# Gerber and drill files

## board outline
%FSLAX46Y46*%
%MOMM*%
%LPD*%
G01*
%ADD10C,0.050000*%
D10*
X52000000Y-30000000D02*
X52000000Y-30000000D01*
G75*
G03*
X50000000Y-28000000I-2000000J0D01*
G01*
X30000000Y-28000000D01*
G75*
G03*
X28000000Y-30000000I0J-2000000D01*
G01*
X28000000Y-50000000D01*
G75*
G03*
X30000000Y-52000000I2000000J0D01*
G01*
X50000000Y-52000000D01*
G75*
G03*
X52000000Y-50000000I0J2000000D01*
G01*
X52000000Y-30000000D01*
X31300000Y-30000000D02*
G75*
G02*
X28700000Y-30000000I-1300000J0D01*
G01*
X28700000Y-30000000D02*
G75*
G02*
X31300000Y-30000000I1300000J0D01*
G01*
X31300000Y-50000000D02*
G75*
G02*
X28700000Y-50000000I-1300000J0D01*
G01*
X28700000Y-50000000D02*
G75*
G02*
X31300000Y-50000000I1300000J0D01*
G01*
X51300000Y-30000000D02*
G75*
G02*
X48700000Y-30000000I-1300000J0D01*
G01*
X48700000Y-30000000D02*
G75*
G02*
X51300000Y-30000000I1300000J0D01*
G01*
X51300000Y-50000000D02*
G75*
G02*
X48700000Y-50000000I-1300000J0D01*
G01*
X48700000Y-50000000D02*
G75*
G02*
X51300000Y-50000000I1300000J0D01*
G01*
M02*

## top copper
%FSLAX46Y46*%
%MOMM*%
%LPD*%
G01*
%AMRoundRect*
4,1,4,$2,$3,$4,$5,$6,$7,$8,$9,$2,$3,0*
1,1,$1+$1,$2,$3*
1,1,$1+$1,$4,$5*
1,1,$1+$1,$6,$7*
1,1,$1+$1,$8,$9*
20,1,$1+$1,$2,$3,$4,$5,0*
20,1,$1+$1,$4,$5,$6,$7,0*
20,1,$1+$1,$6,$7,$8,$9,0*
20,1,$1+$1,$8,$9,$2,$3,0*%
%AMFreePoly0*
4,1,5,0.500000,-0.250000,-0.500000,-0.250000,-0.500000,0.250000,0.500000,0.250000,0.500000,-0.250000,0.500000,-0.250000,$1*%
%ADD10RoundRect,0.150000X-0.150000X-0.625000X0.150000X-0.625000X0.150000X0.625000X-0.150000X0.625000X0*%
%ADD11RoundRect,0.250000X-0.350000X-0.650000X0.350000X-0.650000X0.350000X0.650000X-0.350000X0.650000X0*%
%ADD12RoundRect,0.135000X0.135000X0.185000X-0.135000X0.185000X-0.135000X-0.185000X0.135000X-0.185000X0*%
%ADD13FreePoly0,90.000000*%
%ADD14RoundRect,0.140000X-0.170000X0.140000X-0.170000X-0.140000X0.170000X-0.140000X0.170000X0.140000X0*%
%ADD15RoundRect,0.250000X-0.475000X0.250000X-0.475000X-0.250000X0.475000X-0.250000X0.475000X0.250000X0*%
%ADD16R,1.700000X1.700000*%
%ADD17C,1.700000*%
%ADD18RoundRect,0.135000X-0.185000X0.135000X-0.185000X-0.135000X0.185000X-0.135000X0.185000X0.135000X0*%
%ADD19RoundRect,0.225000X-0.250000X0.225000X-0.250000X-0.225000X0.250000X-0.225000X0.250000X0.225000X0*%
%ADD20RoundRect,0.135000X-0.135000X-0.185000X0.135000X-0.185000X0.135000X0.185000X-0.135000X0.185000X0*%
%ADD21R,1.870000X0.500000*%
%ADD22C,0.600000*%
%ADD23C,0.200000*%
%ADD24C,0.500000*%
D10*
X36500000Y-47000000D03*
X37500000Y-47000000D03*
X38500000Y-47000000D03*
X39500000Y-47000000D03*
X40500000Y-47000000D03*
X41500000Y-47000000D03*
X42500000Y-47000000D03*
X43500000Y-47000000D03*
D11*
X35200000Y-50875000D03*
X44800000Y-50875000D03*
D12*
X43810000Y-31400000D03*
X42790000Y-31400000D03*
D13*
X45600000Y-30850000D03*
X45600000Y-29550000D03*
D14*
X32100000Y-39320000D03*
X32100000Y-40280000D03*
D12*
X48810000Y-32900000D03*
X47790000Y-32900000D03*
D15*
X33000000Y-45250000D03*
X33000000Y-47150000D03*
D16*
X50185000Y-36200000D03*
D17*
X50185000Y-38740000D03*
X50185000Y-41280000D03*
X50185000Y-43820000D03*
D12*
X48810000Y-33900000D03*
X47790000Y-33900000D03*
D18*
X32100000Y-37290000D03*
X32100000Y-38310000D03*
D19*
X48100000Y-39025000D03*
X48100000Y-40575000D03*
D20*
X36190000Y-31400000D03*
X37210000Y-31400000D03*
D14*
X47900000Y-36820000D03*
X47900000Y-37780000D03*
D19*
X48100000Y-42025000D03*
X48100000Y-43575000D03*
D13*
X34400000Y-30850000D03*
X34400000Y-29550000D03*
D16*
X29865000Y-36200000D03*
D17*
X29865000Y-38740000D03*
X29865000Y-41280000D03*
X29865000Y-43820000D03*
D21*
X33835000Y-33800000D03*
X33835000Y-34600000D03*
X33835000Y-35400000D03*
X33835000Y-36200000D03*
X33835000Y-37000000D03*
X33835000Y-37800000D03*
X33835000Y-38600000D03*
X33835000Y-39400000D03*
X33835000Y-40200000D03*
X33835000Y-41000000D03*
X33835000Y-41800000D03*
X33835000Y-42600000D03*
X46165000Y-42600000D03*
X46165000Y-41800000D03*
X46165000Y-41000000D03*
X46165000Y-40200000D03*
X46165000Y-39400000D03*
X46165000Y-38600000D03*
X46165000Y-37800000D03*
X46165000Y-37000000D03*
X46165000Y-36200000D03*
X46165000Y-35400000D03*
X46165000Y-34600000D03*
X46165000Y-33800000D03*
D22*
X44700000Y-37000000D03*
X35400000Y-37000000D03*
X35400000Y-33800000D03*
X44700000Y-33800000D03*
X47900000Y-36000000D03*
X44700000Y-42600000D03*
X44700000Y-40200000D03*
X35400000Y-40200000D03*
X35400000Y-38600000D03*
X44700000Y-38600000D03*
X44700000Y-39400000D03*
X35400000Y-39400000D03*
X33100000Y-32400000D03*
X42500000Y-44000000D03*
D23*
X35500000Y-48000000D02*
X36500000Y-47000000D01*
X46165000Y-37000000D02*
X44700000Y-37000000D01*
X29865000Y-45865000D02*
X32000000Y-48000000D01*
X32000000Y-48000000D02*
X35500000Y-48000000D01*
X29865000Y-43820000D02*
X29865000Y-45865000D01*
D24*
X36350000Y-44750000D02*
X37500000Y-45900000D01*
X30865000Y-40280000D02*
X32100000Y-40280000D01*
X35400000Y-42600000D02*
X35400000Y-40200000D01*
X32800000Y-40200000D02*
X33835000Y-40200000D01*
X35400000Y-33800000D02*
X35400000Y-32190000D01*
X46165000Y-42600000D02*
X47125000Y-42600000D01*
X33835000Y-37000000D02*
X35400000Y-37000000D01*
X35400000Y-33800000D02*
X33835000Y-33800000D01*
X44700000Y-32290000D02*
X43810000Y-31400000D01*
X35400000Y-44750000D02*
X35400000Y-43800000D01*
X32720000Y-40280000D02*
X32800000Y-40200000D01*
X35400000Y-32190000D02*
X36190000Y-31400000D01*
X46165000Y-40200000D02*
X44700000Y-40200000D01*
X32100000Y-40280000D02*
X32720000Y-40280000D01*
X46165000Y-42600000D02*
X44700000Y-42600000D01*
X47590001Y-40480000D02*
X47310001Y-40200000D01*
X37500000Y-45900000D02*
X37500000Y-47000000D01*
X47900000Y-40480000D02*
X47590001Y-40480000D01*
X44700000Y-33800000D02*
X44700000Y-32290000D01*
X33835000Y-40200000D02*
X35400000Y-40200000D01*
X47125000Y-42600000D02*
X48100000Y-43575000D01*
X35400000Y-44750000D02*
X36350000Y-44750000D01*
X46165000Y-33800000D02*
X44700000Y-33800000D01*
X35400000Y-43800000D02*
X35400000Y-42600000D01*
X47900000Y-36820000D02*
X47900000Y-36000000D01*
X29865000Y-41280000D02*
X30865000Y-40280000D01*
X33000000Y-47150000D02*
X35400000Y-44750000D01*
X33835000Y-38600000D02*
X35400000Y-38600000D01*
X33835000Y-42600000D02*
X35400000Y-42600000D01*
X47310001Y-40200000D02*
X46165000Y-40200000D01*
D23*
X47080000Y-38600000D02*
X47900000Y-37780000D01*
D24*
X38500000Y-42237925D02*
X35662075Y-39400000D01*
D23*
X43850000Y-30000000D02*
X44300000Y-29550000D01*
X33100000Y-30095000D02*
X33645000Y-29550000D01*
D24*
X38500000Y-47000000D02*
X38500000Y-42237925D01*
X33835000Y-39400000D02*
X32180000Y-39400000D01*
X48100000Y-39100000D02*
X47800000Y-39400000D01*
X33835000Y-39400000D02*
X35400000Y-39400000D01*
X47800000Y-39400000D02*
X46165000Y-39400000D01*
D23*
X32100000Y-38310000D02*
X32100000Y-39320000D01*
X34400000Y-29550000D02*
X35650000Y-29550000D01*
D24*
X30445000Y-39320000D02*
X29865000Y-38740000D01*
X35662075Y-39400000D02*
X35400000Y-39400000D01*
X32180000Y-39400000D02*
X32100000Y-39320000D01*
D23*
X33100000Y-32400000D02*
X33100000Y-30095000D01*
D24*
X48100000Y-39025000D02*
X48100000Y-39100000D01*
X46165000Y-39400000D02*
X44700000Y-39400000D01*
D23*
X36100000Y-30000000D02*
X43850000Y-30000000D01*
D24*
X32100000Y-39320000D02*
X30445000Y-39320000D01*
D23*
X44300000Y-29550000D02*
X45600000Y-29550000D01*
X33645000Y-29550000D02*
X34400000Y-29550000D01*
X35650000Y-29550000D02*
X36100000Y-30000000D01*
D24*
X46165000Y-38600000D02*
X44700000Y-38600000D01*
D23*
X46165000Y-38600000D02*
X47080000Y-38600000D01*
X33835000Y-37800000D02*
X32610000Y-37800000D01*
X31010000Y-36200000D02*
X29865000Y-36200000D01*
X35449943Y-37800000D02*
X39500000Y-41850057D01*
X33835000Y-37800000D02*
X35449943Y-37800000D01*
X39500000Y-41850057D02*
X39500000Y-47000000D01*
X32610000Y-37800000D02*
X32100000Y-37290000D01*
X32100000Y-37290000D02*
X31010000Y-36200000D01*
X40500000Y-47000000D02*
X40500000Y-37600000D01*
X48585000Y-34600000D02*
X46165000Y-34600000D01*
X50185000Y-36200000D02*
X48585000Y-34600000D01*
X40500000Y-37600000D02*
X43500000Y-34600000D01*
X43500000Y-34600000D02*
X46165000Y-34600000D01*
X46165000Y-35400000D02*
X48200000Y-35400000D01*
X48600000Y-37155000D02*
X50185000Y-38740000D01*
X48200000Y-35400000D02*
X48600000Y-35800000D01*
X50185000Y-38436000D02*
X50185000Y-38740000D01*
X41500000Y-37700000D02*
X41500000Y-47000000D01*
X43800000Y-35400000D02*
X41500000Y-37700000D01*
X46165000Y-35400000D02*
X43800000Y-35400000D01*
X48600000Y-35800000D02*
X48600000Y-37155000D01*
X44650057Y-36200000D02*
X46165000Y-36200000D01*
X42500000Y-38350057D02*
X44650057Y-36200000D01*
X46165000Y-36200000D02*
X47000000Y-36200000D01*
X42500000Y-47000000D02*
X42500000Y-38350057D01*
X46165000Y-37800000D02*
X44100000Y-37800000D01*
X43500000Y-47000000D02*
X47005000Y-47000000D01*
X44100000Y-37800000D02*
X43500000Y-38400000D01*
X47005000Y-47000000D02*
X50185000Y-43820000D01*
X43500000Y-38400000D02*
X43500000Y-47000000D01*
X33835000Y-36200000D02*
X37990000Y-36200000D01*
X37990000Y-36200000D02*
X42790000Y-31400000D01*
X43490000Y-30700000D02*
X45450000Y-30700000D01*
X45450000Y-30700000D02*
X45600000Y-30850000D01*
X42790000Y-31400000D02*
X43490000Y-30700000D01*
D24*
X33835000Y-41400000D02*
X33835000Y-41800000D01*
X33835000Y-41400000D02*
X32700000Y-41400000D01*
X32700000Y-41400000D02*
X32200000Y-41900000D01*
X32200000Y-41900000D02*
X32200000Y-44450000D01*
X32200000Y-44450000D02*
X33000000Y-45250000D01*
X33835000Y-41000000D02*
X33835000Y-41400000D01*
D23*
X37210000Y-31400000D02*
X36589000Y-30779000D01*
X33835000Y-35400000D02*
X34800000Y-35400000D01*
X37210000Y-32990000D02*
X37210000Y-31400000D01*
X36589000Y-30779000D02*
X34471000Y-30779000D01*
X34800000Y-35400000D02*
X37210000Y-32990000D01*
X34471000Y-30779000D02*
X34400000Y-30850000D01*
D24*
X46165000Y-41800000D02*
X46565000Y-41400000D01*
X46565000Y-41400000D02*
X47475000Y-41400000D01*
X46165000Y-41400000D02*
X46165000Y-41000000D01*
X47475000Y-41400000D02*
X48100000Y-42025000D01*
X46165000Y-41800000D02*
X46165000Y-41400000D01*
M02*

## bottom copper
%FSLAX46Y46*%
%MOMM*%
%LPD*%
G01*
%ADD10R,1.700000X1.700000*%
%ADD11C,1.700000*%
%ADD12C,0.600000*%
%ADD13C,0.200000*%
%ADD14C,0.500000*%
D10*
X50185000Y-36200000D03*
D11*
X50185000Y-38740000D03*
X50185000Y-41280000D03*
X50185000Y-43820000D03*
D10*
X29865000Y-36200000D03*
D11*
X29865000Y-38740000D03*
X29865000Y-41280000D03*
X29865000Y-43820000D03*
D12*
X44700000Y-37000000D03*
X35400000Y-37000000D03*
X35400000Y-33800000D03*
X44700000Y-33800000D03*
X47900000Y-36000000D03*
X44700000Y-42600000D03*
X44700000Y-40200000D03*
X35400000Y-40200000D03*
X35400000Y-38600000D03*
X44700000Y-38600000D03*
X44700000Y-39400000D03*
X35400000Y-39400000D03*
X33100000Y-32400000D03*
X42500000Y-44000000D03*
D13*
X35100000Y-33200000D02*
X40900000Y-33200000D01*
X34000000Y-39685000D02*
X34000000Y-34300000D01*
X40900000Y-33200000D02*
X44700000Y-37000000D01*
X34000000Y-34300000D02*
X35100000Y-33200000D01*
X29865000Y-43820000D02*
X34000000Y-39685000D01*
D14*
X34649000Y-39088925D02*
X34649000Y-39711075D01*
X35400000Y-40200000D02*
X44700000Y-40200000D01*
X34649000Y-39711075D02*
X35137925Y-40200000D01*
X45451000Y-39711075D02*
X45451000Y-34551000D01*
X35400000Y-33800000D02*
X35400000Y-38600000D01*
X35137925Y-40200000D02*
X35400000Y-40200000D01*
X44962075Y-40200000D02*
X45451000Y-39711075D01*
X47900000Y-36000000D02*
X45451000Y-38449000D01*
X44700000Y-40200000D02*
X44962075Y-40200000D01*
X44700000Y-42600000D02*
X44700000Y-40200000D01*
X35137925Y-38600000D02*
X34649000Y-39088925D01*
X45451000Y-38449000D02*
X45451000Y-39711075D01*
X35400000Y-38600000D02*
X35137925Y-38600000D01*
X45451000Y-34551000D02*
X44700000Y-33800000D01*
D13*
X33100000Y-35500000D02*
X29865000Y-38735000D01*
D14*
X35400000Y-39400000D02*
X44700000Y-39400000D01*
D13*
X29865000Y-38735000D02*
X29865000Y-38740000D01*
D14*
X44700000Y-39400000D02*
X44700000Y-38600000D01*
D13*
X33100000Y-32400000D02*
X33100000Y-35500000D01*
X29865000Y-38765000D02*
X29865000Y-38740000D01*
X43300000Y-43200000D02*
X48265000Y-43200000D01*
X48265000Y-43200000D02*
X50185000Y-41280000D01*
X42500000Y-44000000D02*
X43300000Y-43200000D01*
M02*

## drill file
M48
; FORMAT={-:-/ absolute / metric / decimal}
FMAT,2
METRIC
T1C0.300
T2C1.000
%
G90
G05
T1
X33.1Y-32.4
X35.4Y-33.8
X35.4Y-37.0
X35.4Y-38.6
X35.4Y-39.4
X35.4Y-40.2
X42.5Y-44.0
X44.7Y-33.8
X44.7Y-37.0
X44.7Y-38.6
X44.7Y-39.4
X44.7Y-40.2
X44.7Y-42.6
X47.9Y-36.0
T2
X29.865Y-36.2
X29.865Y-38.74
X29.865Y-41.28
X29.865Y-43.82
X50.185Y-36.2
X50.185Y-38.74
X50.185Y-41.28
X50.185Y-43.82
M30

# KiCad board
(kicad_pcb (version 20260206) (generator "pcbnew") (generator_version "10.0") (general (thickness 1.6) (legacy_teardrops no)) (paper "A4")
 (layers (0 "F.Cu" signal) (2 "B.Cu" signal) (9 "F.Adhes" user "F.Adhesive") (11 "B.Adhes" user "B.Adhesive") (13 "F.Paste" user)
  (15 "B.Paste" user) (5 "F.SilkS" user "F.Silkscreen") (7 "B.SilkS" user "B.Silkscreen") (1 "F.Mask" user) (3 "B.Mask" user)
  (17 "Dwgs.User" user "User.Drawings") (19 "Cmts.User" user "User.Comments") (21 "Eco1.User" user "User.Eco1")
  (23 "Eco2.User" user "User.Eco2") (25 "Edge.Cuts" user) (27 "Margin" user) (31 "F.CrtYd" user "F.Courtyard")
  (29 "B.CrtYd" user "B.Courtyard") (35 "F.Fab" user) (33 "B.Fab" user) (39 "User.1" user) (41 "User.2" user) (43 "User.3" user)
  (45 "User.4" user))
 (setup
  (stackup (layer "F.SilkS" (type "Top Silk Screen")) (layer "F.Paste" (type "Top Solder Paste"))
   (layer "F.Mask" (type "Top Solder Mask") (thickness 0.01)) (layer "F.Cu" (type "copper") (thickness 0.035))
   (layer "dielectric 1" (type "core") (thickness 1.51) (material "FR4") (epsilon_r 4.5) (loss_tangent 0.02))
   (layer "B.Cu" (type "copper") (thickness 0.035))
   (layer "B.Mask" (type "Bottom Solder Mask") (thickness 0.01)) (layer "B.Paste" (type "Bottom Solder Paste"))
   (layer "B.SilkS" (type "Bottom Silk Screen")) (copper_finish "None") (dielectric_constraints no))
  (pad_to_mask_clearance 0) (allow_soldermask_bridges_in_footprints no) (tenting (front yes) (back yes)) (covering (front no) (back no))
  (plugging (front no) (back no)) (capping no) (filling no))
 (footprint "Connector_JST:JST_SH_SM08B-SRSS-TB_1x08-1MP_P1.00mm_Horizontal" (layer "F.Cu") (at 40 49)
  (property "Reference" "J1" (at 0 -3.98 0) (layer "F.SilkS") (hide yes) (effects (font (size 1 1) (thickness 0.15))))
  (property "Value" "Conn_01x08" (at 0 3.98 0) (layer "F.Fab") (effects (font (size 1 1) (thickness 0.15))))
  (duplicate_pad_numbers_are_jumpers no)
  (pad "1" smd roundrect (at -3.5 -2) (size 0.6 1.55) (layers "F.Cu" "F.Mask" "F.Paste") (roundrect_rratio 0.25) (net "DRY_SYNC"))
  (pad "2" smd roundrect (at -2.5 -2) (size 0.6 1.55) (layers "F.Cu" "F.Mask" "F.Paste") (roundrect_rratio 0.25) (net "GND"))
  (pad "3" smd roundrect (at -1.5 -2) (size 0.6 1.55) (layers "F.Cu" "F.Mask" "F.Paste") (roundrect_rratio 0.25) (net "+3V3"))
  (pad "4" smd roundrect (at -0.5 -2) (size 0.6 1.55) (layers "F.Cu" "F.Mask" "F.Paste") (roundrect_rratio 0.25) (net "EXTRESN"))
  (pad "5" smd roundrect (at 0.5 -2) (size 0.6 1.55) (layers "F.Cu" "F.Mask" "F.Paste") (roundrect_rratio 0.25) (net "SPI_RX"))
  (pad "6" smd roundrect (at 1.5 -2) (size 0.6 1.55) (layers "F.Cu" "F.Mask" "F.Paste") (roundrect_rratio 0.25) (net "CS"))
  (pad "7" smd roundrect (at 2.5 -2) (size 0.6 1.55) (layers "F.Cu" "F.Mask" "F.Paste") (roundrect_rratio 0.25) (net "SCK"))
  (pad "8" smd roundrect (at 3.5 -2) (size 0.6 1.55) (layers "F.Cu" "F.Mask" "F.Paste") (roundrect_rratio 0.25) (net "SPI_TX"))
  (pad "MP" smd roundrect (at -4.8 1.875) (size 1.2 1.8) (layers "F.Cu" "F.Mask" "F.Paste") (roundrect_rratio 0.208333))
  (pad "MP" smd roundrect (at 4.8 1.875) (size 1.2 1.8) (layers "F.Cu" "F.Mask" "F.Paste") (roundrect_rratio 0.208333)))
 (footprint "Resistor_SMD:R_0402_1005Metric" (layer "F.Cu") (at 43.3 31.4 180)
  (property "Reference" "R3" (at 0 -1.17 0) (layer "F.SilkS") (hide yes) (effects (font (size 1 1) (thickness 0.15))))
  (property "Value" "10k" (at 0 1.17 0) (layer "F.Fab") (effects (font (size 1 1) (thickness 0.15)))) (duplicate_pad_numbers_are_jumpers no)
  (pad "1" smd roundrect (at -0.51 0 180) (size 0.54 0.64) (layers "F.Cu" "F.Mask" "F.Paste") (roundrect_rratio 0.25) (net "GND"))
  (pad "2" smd roundrect (at 0.51 0 180) (size 0.54 0.64) (layers "F.Cu" "F.Mask" "F.Paste") (roundrect_rratio 0.25) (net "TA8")))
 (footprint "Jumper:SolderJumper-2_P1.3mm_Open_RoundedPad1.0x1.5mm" (layer "F.Cu") (at 45.6 30.2 90)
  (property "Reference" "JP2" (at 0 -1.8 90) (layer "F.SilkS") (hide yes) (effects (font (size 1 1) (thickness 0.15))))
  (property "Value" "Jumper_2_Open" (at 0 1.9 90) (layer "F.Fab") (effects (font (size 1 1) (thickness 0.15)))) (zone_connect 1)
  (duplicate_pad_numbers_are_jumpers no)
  (pad "1" smd custom (at -0.65 0 90) (size 1 0.5) (layers "F.Cu" "F.Mask") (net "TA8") (zone_connect 2) (thermal_bridge_angle 45)
   (options (clearance outline) (anchor rect)) (primitives))
  (pad "2" smd custom (at 0.65 0 90) (size 1 0.5) (layers "F.Cu" "F.Mask") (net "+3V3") (zone_connect 2) (thermal_bridge_angle 45)
   (options (clearance outline) (anchor rect)) (primitives)))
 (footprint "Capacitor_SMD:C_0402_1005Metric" (layer "F.Cu") (at 32.1 39.8 -90)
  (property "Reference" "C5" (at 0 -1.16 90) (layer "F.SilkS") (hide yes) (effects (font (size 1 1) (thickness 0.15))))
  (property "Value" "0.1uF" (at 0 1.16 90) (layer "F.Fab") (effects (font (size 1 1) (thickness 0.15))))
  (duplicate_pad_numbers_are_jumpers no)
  (pad "1" smd roundrect (at -0.48 0 270) (size 0.56 0.62) (layers "F.Cu" "F.Mask" "F.Paste") (roundrect_rratio 0.25) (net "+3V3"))
  (pad "2" smd roundrect (at 0.48 0 270) (size 0.56 0.62) (layers "F.Cu" "F.Mask" "F.Paste") (roundrect_rratio 0.25) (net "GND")))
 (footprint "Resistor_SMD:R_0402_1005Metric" (layer "F.Cu") (at 48.3 32.9 180)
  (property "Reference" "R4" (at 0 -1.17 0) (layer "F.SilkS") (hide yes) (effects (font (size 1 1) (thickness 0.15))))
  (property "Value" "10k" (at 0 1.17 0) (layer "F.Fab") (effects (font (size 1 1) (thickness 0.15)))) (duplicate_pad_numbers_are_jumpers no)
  (pad "1" smd roundrect (at -0.51 0 180) (size 0.54 0.64) (layers "F.Cu" "F.Mask" "F.Paste") (roundrect_rratio 0.25)
   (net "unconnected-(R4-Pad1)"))
  (pad "2" smd roundrect (at 0.51 0 180) (size 0.54 0.64) (layers "F.Cu" "F.Mask" "F.Paste") (roundrect_rratio 0.25)
   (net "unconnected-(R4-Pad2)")))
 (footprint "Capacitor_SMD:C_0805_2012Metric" (layer "F.Cu") (at 33 46.2 -90)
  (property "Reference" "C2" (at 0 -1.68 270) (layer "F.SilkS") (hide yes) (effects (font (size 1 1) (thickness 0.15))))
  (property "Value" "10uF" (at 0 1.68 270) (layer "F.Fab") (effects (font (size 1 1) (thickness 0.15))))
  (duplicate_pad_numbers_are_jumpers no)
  (pad "1" smd roundrect (at -0.95 0 270) (size 1 1.45) (layers "F.Cu" "F.Mask" "F.Paste") (roundrect_rratio 0.25) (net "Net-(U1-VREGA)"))
  (pad "2" smd roundrect (at 0.95 0 270) (size 1 1.45) (layers "F.Cu" "F.Mask" "F.Paste") (roundrect_rratio 0.25) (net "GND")))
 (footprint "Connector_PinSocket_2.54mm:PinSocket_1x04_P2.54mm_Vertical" (layer "F.Cu") (at 50.185 36.2)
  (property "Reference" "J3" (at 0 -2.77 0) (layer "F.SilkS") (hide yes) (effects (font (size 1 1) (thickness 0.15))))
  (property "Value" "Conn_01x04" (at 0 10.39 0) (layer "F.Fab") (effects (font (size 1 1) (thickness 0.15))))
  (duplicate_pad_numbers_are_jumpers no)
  (pad "1" thru_hole rect (at 0 0) (size 1.7 1.7) (drill 1) (layers "*.Cu" "*.Mask") (remove_unused_layers no) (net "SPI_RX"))
  (pad "2" thru_hole circle (at 0 2.54) (size 1.7 1.7) (drill 1) (layers "*.Cu" "*.Mask") (remove_unused_layers no) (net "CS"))
  (pad "3" thru_hole circle (at 0 5.08) (size 1.7 1.7) (drill 1) (layers "*.Cu" "*.Mask") (remove_unused_layers no) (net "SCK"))
  (pad "4" thru_hole circle (at 0 7.62) (size 1.7 1.7) (drill 1) (layers "*.Cu" "*.Mask") (remove_unused_layers no) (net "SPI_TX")))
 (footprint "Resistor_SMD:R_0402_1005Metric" (layer "F.Cu") (at 48.3 33.9 180)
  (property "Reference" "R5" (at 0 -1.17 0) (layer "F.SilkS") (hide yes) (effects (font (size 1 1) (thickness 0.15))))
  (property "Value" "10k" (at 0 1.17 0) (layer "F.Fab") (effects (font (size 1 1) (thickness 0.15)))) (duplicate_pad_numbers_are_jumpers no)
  (pad "1" smd roundrect (at -0.51 0 180) (size 0.54 0.64) (layers "F.Cu" "F.Mask" "F.Paste") (roundrect_rratio 0.25)
   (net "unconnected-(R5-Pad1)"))
  (pad "2" smd roundrect (at 0.51 0 180) (size 0.54 0.64) (layers "F.Cu" "F.Mask" "F.Paste") (roundrect_rratio 0.25)
   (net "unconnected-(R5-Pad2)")))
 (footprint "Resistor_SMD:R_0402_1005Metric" (layer "F.Cu") (at 32.1 37.8 -90)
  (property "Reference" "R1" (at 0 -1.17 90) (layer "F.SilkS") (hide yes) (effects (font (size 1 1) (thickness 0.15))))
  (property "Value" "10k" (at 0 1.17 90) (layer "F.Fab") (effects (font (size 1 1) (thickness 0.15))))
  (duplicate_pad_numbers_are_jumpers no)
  (pad "1" smd roundrect (at -0.51 0 270) (size 0.54 0.64) (layers "F.Cu" "F.Mask" "F.Paste") (roundrect_rratio 0.25) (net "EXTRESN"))
  (pad "2" smd roundrect (at 0.51 0 270) (size 0.54 0.64) (layers "F.Cu" "F.Mask" "F.Paste") (roundrect_rratio 0.25) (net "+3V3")))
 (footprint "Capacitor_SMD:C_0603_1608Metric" (layer "F.Cu") (at 48.1 39.8 -90)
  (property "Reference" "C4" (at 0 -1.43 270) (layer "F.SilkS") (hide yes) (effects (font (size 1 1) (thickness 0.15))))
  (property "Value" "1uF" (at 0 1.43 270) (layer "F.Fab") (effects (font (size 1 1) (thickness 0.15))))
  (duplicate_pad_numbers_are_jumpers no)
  (pad "1" smd roundrect (at -0.775 0 270) (size 0.9 0.95) (layers "F.Cu" "F.Mask" "F.Paste") (roundrect_rratio 0.25) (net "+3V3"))
  (pad "2" smd roundrect (at 0.775 0 270) (size 0.9 0.95) (layers "F.Cu" "F.Mask" "F.Paste") (roundrect_rratio 0.25) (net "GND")))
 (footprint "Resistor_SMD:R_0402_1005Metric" (layer "F.Cu") (at 36.7 31.4)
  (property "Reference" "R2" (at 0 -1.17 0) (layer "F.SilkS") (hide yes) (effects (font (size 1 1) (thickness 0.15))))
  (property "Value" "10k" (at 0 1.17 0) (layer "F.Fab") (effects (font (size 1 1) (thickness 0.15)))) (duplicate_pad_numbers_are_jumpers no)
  (pad "1" smd roundrect (at -0.51 0) (size 0.54 0.64) (layers "F.Cu" "F.Mask" "F.Paste") (roundrect_rratio 0.25) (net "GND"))
  (pad "2" smd roundrect (at 0.51 0) (size 0.54 0.64) (layers "F.Cu" "F.Mask" "F.Paste") (roundrect_rratio 0.25) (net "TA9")))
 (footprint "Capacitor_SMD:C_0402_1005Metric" (layer "F.Cu") (at 47.9 37.3 -90)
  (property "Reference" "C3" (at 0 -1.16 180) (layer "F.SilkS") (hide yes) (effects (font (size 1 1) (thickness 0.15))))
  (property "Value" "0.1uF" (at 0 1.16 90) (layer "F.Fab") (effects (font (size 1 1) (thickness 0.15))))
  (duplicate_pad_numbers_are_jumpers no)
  (pad "1" smd roundrect (at -0.48 0 270) (size 0.56 0.62) (layers "F.Cu" "F.Mask" "F.Paste") (roundrect_rratio 0.25) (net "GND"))
  (pad "2" smd roundrect (at 0.48 0 270) (size 0.56 0.62) (layers "F.Cu" "F.Mask" "F.Paste") (roundrect_rratio 0.25) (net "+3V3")))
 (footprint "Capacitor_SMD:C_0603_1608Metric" (layer "F.Cu") (at 48.1 42.8 -90)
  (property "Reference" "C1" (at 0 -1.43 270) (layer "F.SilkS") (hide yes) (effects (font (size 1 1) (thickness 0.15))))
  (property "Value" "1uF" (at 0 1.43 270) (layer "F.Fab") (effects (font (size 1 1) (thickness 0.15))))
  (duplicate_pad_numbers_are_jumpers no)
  (pad "1" smd roundrect (at -0.775 0 270) (size 0.9 0.95) (layers "F.Cu" "F.Mask" "F.Paste") (roundrect_rratio 0.25) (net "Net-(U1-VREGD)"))
  (pad "2" smd roundrect (at 0.775 0 270) (size 0.9 0.95) (layers "F.Cu" "F.Mask" "F.Paste") (roundrect_rratio 0.25) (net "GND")))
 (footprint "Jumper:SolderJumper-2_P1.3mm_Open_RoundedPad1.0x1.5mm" (layer "F.Cu") (at 34.4 30.2 90)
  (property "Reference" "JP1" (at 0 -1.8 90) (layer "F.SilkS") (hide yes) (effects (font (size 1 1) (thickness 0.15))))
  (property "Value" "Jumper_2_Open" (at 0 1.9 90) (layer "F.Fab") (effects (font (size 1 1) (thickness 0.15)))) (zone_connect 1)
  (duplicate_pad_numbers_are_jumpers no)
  (pad "1" smd custom (at -0.65 0 90) (size 1 0.5) (layers "F.Cu" "F.Mask") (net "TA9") (zone_connect 2) (thermal_bridge_angle 45)
   (options (clearance outline) (anchor rect)) (primitives))
  (pad "2" smd custom (at 0.65 0 90) (size 1 0.5) (layers "F.Cu" "F.Mask") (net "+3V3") (zone_connect 2) (thermal_bridge_angle 45)
   (options (clearance outline) (anchor rect)) (primitives)))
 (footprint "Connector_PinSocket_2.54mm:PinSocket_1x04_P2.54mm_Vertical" (layer "F.Cu") (at 29.865 36.2)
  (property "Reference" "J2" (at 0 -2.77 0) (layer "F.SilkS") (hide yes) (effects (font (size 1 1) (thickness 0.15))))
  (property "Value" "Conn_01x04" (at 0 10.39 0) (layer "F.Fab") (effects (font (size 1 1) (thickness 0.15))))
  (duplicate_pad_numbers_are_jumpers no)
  (pad "1" thru_hole rect (at 0 0) (size 1.7 1.7) (drill 1) (layers "*.Cu" "*.Mask") (remove_unused_layers no) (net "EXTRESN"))
  (pad "2" thru_hole circle (at 0 2.54) (size 1.7 1.7) (drill 1) (layers "*.Cu" "*.Mask") (remove_unused_layers no) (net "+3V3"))
  (pad "3" thru_hole circle (at 0 5.08) (size 1.7 1.7) (drill 1) (layers "*.Cu" "*.Mask") (remove_unused_layers no) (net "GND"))
  (pad "4" thru_hole circle (at 0 7.62) (size 1.7 1.7) (drill 1) (layers "*.Cu" "*.Mask") (remove_unused_layers no) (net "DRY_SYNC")))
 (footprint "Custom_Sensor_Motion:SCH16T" (layer "F.Cu") (at 40 38.2)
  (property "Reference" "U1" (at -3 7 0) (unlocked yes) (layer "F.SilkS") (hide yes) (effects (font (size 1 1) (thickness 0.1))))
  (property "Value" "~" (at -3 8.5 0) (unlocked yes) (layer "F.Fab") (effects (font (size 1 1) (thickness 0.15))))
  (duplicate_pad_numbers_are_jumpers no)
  (pad "1" smd rect (at -6.165 -4.4) (size 1.87 0.5) (layers "F.Cu" "F.Mask" "F.Paste") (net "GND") (thermal_bridge_angle 45))
  (pad "2" smd rect (at -6.165 -3.6) (size 1.87 0.5) (layers "F.Cu" "F.Mask" "F.Paste") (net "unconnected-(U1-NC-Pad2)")
   (thermal_bridge_angle 45))
  (pad "3" smd rect (at -6.165 -2.8) (size 1.87 0.5) (layers "F.Cu" "F.Mask" "F.Paste") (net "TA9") (thermal_bridge_angle 45))
  (pad "4" smd rect (at -6.165 -2) (size 1.87 0.5) (layers "F.Cu" "F.Mask" "F.Paste") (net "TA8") (thermal_bridge_angle 45))
  (pad "5" smd rect (at -6.165 -1.2) (size 1.87 0.5) (layers "F.Cu" "F.Mask" "F.Paste") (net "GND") (thermal_bridge_angle 45))
  (pad "6" smd rect (at -6.165 -0.4) (size 1.87 0.5) (layers "F.Cu" "F.Mask" "F.Paste") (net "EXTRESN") (thermal_bridge_angle 45))
  (pad "7" smd rect (at -6.165 0.4) (size 1.87 0.5) (layers "F.Cu" "F.Mask" "F.Paste") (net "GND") (thermal_bridge_angle 45))
  (pad "8" smd rect (at -6.165 1.2) (size 1.87 0.5) (layers "F.Cu" "F.Mask" "F.Paste") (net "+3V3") (thermal_bridge_angle 45))
  (pad "9" smd rect (at -6.165 2) (size 1.87 0.5) (layers "F.Cu" "F.Mask" "F.Paste") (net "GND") (thermal_bridge_angle 45))
  (pad "10" smd rect (at -6.165 2.8) (size 1.87 0.5) (layers "F.Cu" "F.Mask" "F.Paste") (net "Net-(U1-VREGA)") (thermal_bridge_angle 45))
  (pad "11" smd rect (at -6.165 3.6) (size 1.87 0.5) (layers "F.Cu" "F.Mask" "F.Paste") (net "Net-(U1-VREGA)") (thermal_bridge_angle 45))
  (pad "12" smd rect (at -6.165 4.4) (size 1.87 0.5) (layers "F.Cu" "F.Mask" "F.Paste") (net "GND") (thermal_bridge_angle 45))
  (pad "13" smd rect (at 6.165 4.4) (size 1.87 0.5) (layers "F.Cu" "F.Mask" "F.Paste") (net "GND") (thermal_bridge_angle 45))
  (pad "14" smd rect (at 6.165 3.6) (size 1.87 0.5) (layers "F.Cu" "F.Mask" "F.Paste") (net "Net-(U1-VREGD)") (thermal_bridge_angle 45))
  (pad "15" smd rect (at 6.165 2.8) (size 1.87 0.5) (layers "F.Cu" "F.Mask" "F.Paste") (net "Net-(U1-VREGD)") (thermal_bridge_angle 45))
  (pad "16" smd rect (at 6.165 2) (size 1.87 0.5) (layers "F.Cu" "F.Mask" "F.Paste") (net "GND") (thermal_bridge_angle 45))
  (pad "17" smd rect (at 6.165 1.2) (size 1.87 0.5) (layers "F.Cu" "F.Mask" "F.Paste") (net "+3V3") (thermal_bridge_angle 45))
  (pad "18" smd rect (at 6.165 0.4) (size 1.87 0.5) (layers "F.Cu" "F.Mask" "F.Paste") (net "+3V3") (thermal_bridge_angle 45))
  (pad "19" smd rect (at 6.165 -0.4) (size 1.87 0.5) (layers "F.Cu" "F.Mask" "F.Paste") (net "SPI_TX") (thermal_bridge_angle 45))
  (pad "20" smd rect (at 6.165 -1.2) (size 1.87 0.5) (layers "F.Cu" "F.Mask" "F.Paste") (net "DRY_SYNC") (thermal_bridge_angle 45))
  (pad "21" smd rect (at 6.165 -2) (size 1.87 0.5) (layers "F.Cu" "F.Mask" "F.Paste") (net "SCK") (thermal_bridge_angle 45))
  (pad "22" smd rect (at 6.165 -2.8) (size 1.87 0.5) (layers "F.Cu" "F.Mask" "F.Paste") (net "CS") (thermal_bridge_angle 45))
  (pad "23" smd rect (at 6.165 -3.6) (size 1.87 0.5) (layers "F.Cu" "F.Mask" "F.Paste") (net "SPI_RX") (thermal_bridge_angle 45))
  (pad "24" smd rect (at 6.165 -4.4) (size 1.87 0.5) (layers "F.Cu" "F.Mask" "F.Paste") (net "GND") (thermal_bridge_angle 45)))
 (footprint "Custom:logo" (layer "B.Cu") (at 40 32 180)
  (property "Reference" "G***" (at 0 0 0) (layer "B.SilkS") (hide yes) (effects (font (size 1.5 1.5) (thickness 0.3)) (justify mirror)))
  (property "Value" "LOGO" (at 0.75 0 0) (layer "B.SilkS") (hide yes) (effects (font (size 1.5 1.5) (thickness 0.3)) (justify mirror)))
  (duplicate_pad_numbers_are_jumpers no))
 (gr_poly
  (pts (arc (start 52 30) (mid 51.414214 28.585786) (end 50 28)) (arc (start 30 28) (mid 28.585786 28.585786) (end 28 30))
   (arc (start 28 50) (mid 28.585786 51.414214) (end 30 52)) (arc (start 50 52) (mid 51.414214 51.414214) (end 52 50)))
  (stroke (width 0.05) (type solid)) (fill no) (layer "Edge.Cuts"))
 (gr_circle (center 30 30) (end 31.3 30) (stroke (width 0.05) (type solid)) (fill no) (layer "Edge.Cuts"))
 (gr_circle (center 30 50) (end 31.3 50) (stroke (width 0.05) (type solid)) (fill no) (layer "Edge.Cuts"))
 (gr_circle (center 50 30) (end 51.3 30) (stroke (width 0.05) (type solid)) (fill no) (layer "Edge.Cuts"))
 (gr_circle (center 50 50) (end 51.3 50) (stroke (width 0.05) (type solid)) (fill no) (layer "Edge.Cuts"))
 (segment (start 35.5 48) (end 36.5 47) (width 0.2) (layer "F.Cu") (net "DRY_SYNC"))
 (segment (start 46.165 37) (end 44.7 37) (width 0.2) (layer "F.Cu") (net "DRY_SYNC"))
 (segment (start 29.865 45.865) (end 32 48) (width 0.2) (layer "F.Cu") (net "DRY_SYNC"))
 (segment (start 32 48) (end 35.5 48) (width 0.2) (layer "F.Cu") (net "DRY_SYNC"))
 (segment (start 29.865 43.82) (end 29.865 45.865) (width 0.2) (layer "F.Cu") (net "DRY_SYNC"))
 (via (at 44.7 37) (size 0.6) (drill 0.3) (layers "F.Cu" "B.Cu") (capping no) (covering (front no) (back no))
  (plugging (front no) (back no)) (filling no) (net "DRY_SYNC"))
 (segment (start 35.1 33.2) (end 40.9 33.2) (width 0.2) (layer "B.Cu") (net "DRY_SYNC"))
 (segment (start 34 39.685) (end 34 34.3) (width 0.2) (layer "B.Cu") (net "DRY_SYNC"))
 (segment (start 40.9 33.2) (end 44.7 37) (width 0.2) (layer "B.Cu") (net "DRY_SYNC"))
 (segment (start 34 34.3) (end 35.1 33.2) (width 0.2) (layer "B.Cu") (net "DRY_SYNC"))
 (segment (start 29.865 43.82) (end 34 39.685) (width 0.2) (layer "B.Cu") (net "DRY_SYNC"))
 (segment (start 36.35 44.75) (end 37.5 45.9) (width 0.5) (layer "F.Cu") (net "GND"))
 (segment (start 30.865 40.28) (end 32.1 40.28) (width 0.5) (layer "F.Cu") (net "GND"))
 (segment (start 35.4 42.6) (end 35.4 40.2) (width 0.5) (layer "F.Cu") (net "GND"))
 (segment (start 32.8 40.2) (end 33.835 40.2) (width 0.5) (layer "F.Cu") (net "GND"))
 (segment (start 35.4 33.8) (end 35.4 32.19) (width 0.5) (layer "F.Cu") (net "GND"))
 (segment (start 46.165 42.6) (end 47.125 42.6) (width 0.5) (layer "F.Cu") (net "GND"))
 (segment (start 33.835 37) (end 35.4 37) (width 0.5) (layer "F.Cu") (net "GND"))
 (segment (start 35.4 33.8) (end 33.835 33.8) (width 0.5) (layer "F.Cu") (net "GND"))
 (segment (start 44.7 32.29) (end 43.81 31.4) (width 0.5) (layer "F.Cu") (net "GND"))
 (segment (start 35.4 44.75) (end 35.4 43.8) (width 0.5) (layer "F.Cu") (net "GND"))
 (segment (start 32.72 40.28) (end 32.8 40.2) (width 0.5) (layer "F.Cu") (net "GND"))
 (segment (start 35.4 32.19) (end 36.19 31.4) (width 0.5) (layer "F.Cu") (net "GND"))
 (segment (start 46.165 40.2) (end 44.7 40.2) (width 0.5) (layer "F.Cu") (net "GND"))
 (segment (start 32.1 40.28) (end 32.72 40.28) (width 0.5) (layer "F.Cu") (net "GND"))
 (segment (start 46.165 42.6) (end 44.7 42.6) (width 0.5) (layer "F.Cu") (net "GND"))
 (segment (start 47.590001 40.48) (end 47.310001 40.2) (width 0.5) (layer "F.Cu") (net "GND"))
 (segment (start 37.5 45.9) (end 37.5 47) (width 0.5) (layer "F.Cu") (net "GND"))
 (segment (start 47.9 40.48) (end 47.590001 40.48) (width 0.5) (layer "F.Cu") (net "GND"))
 (segment (start 44.7 33.8) (end 44.7 32.29) (width 0.5) (layer "F.Cu") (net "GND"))
 (segment (start 33.835 40.2) (end 35.4 40.2) (width 0.5) (layer "F.Cu") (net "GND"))
 (segment (start 47.125 42.6) (end 48.1 43.575) (width 0.5) (layer "F.Cu") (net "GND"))
 (segment (start 35.4 44.75) (end 36.35 44.75) (width 0.5) (layer "F.Cu") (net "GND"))
 (segment (start 46.165 33.8) (end 44.7 33.8) (width 0.5) (layer "F.Cu") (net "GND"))
 (segment (start 35.4 43.8) (end 35.4 42.6) (width 0.5) (layer "F.Cu") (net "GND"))
 (segment (start 47.9 36.82) (end 47.9 36) (width 0.5) (layer "F.Cu") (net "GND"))
 (segment (start 29.865 41.28) (end 30.865 40.28) (width 0.5) (layer "F.Cu") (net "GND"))
 (segment (start 33 47.15) (end 35.4 44.75) (width 0.5) (layer "F.Cu") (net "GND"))
 (segment (start 33.835 38.6) (end 35.4 38.6) (width 0.5) (layer "F.Cu") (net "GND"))
 (segment (start 33.835 42.6) (end 35.4 42.6) (width 0.5) (layer "F.Cu") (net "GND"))
 (segment (start 47.310001 40.2) (end 46.165 40.2) (width 0.5) (layer "F.Cu") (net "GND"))
 (via (at 35.4 37) (size 0.6) (drill 0.3) (layers "F.Cu" "B.Cu") (capping no) (covering (front no) (back no))
  (plugging (front no) (back no)) (filling no) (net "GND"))
 (via (at 35.4 33.8) (size 0.6) (drill 0.3) (layers "F.Cu" "B.Cu") (capping no) (covering (front no) (back no))
  (plugging (front no) (back no)) (filling no) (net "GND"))
 (via (at 44.7 33.8) (size 0.6) (drill 0.3) (layers "F.Cu" "B.Cu") (capping no) (covering (front no) (back no))
  (plugging (front no) (back no)) (filling no) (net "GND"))
 (via (at 47.9 36) (size 0.6) (drill 0.3) (layers "F.Cu" "B.Cu") (capping no) (covering (front no) (back no))
  (plugging (front no) (back no)) (filling no) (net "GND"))
 (via (at 44.7 42.6) (size 0.6) (drill 0.3) (layers "F.Cu" "B.Cu") (capping no) (covering (front no) (back no))
  (plugging (front no) (back no)) (filling no) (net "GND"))
 (via (at 44.7 40.2) (size 0.6) (drill 0.3) (layers "F.Cu" "B.Cu") (capping no) (covering (front no) (back no))
  (plugging (front no) (back no)) (filling no) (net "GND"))
 (via (at 35.4 40.2) (size 0.6) (drill 0.3) (layers "F.Cu" "B.Cu") (capping no) (covering (front no) (back no))
  (plugging (front no) (back no)) (filling no) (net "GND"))
 (via (at 35.4 38.6) (size 0.6) (drill 0.3) (layers "F.Cu" "B.Cu") (capping no) (covering (front no) (back no))
  (plugging (front no) (back no)) (filling no) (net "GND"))
 (segment (start 34.649 39.088925) (end 34.649 39.711075) (width 0.5) (layer "B.Cu") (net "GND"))
 (segment (start 35.4 40.2) (end 44.7 40.2) (width 0.5) (layer "B.Cu") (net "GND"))
 (segment (start 34.649 39.711075) (end 35.137925 40.2) (width 0.5) (layer "B.Cu") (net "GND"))
 (segment (start 45.451 39.711075) (end 45.451 34.551) (width 0.5) (layer "B.Cu") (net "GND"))
 (segment (start 35.4 33.8) (end 35.4 38.6) (width 0.5) (layer "B.Cu") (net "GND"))
 (segment (start 35.137925 40.2) (end 35.4 40.2) (width 0.5) (layer "B.Cu") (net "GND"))
 (segment (start 44.962075 40.2) (end 45.451 39.711075) (width 0.5) (layer "B.Cu") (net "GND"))
 (segment (start 47.9 36) (end 45.451 38.449) (width 0.5) (layer "B.Cu") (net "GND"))
 (segment (start 44.7 40.2) (end 44.962075 40.2) (width 0.5) (layer "B.Cu") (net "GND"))
 (segment (start 44.7 42.6) (end 44.7 40.2) (width 0.5) (layer "B.Cu") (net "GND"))
 (segment (start 35.137925 38.6) (end 34.649 39.088925) (width 0.5) (layer "B.Cu") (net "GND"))
 (segment (start 45.451 38.449) (end 45.451 39.711075) (width 0.5) (layer "B.Cu") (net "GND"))
 (segment (start 35.4 38.6) (end 35.137925 38.6) (width 0.5) (layer "B.Cu") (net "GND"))
 (segment (start 45.451 34.551) (end 44.7 33.8) (width 0.5) (layer "B.Cu") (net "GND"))
 (segment (start 47.08 38.6) (end 47.9 37.78) (width 0.2) (layer "F.Cu") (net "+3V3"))
 (segment (start 38.5 42.237925) (end 35.662075 39.4) (width 0.5) (layer "F.Cu") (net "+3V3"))
 (segment (start 43.85 30) (end 44.3 29.55) (width 0.2) (layer "F.Cu") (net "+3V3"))
 (segment (start 33.1 30.095) (end 33.645 29.55) (width 0.2) (layer "F.Cu") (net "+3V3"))
 (segment (start 38.5 47) (end 38.5 42.237925) (width 0.5) (layer "F.Cu") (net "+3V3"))
 (segment (start 33.835 39.4) (end 32.18 39.4) (width 0.5) (layer "F.Cu") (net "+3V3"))
 (segment (start 48.1 39.1) (end 47.8 39.4) (width 0.5) (layer "F.Cu") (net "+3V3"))
 (segment (start 33.835 39.4) (end 35.4 39.4) (width 0.5) (layer "F.Cu") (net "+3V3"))
 (segment (start 47.8 39.4) (end 46.165 39.4) (width 0.5) (layer "F.Cu") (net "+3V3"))
 (segment (start 32.1 38.31) (end 32.1 39.32) (width 0.2) (layer "F.Cu") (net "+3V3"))
 (segment (start 34.4 29.55) (end 35.65 29.55) (width 0.2) (layer "F.Cu") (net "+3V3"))
 (segment (start 30.445 39.32) (end 29.865 38.74) (width 0.5) (layer "F.Cu") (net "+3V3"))
 (segment (start 35.662075 39.4) (end 35.4 39.4) (width 0.5) (layer "F.Cu") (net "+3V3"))
 (segment (start 32.18 39.4) (end 32.1 39.32) (width 0.5) (layer "F.Cu") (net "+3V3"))
 (segment (start 33.1 32.4) (end 33.1 30.095) (width 0.2) (layer "F.Cu") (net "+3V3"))
 (segment (start 48.1 39.025) (end 48.1 39.1) (width 0.5) (layer "F.Cu") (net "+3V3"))
 (segment (start 46.165 39.4) (end 44.7 39.4) (width 0.5) (layer "F.Cu") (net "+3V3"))
 (segment (start 36.1 30) (end 43.85 30) (width 0.2) (layer "F.Cu") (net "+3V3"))
 (segment (start 32.1 39.32) (end 30.445 39.32) (width 0.5) (layer "F.Cu") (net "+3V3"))
 (segment (start 44.3 29.55) (end 45.6 29.55) (width 0.2) (layer "F.Cu") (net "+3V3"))
 (segment (start 33.645 29.55) (end 34.4 29.55) (width 0.2) (layer "F.Cu") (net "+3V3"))
 (segment (start 35.65 29.55) (end 36.1 30) (width 0.2) (layer "F.Cu") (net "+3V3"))
 (segment (start 46.165 38.6) (end 44.7 38.6) (width 0.5) (layer "F.Cu") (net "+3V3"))
 (segment (start 46.165 38.6) (end 47.08 38.6) (width 0.2) (layer "F.Cu") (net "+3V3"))
 (via (at 44.7 38.6) (size 0.6) (drill 0.3) (layers "F.Cu" "B.Cu") (capping no) (covering (front no) (back no))
  (plugging (front no) (back no)) (filling no) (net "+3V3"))
 (via (at 44.7 39.4) (size 0.6) (drill 0.3) (layers "F.Cu" "B.Cu") (capping no) (covering (front no) (back no))
  (plugging (front no) (back no)) (filling no) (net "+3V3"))
 (via (at 35.4 39.4) (size 0.6) (drill 0.3) (layers "F.Cu" "B.Cu") (capping no) (covering (front no) (back no))
  (plugging (front no) (back no)) (filling no) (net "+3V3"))
 (via (at 33.1 32.4) (size 0.6) (drill 0.3) (layers "F.Cu" "B.Cu") (capping no) (covering (front no) (back no))
  (plugging (front no) (back no)) (filling no) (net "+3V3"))
 (segment (start 33.1 35.5) (end 29.865 38.735) (width 0.2) (layer "B.Cu") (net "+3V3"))
 (segment (start 35.4 39.4) (end 44.7 39.4) (width 0.5) (layer "B.Cu") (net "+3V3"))
 (segment (start 29.865 38.735) (end 29.865 38.74) (width 0.2) (layer "B.Cu") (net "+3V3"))
 (segment (start 44.7 39.4) (end 44.7 38.6) (width 0.5) (layer "B.Cu") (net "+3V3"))
 (segment (start 33.1 32.4) (end 33.1 35.5) (width 0.2) (layer "B.Cu") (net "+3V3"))
 (segment (start 29.865 38.765) (end 29.865 38.74) (width 0.2) (layer "B.Cu") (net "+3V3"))
 (segment (start 33.835 37.8) (end 32.61 37.8) (width 0.2) (layer "F.Cu") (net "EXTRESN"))
 (segment (start 31.01 36.2) (end 29.865 36.2) (width 0.2) (layer "F.Cu") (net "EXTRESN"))
 (segment (start 35.449943 37.8) (end 39.5 41.850057) (width 0.2) (layer "F.Cu") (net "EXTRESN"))
 (segment (start 33.835 37.8) (end 35.449943 37.8) (width 0.2) (layer "F.Cu") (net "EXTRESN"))
 (segment (start 39.5 41.850057) (end 39.5 47) (width 0.2) (layer "F.Cu") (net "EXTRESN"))
 (segment (start 32.61 37.8) (end 32.1 37.29) (width 0.2) (layer "F.Cu") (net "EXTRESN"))
 (segment (start 32.1 37.29) (end 31.01 36.2) (width 0.2) (layer "F.Cu") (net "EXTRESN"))
 (segment (start 40.5 47) (end 40.5 37.6) (width 0.2) (layer "F.Cu") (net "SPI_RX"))
 (segment (start 48.585 34.6) (end 46.165 34.6) (width 0.2) (layer "F.Cu") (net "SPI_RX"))
 (segment (start 50.185 36.2) (end 48.585 34.6) (width 0.2) (layer "F.Cu") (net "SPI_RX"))
 (segment (start 40.5 37.6) (end 43.5 34.6) (width 0.2) (layer "F.Cu") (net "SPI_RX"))
 (segment (start 43.5 34.6) (end 46.165 34.6) (width 0.2) (layer "F.Cu") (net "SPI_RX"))
 (segment (start 46.165 35.4) (end 48.2 35.4) (width 0.2) (layer "F.Cu") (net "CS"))
 (segment (start 48.6 37.155) (end 50.185 38.74) (width 0.2) (layer "F.Cu") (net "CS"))
 (segment (start 48.2 35.4) (end 48.6 35.8) (width 0.2) (layer "F.Cu") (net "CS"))
 (segment (start 50.185 38.436) (end 50.185 38.74) (width 0.2) (layer "F.Cu") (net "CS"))
 (segment (start 41.5 37.7) (end 41.5 47) (width 0.2) (layer "F.Cu") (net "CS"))
 (segment (start 43.8 35.4) (end 41.5 37.7) (width 0.2) (layer "F.Cu") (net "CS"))
 (segment (start 46.165 35.4) (end 43.8 35.4) (width 0.2) (layer "F.Cu") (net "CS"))
 (segment (start 48.6 35.8) (end 48.6 37.155) (width 0.2) (layer "F.Cu") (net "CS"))
 (segment (start 44.650057 36.2) (end 46.165 36.2) (width 0.2) (layer "F.Cu") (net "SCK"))
 (segment (start 42.5 38.350057) (end 44.650057 36.2) (width 0.2) (layer "F.Cu") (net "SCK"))
 (segment (start 46.165 36.2) (end 47 36.2) (width 0.2) (layer "F.Cu") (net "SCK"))
 (segment (start 42.5 47) (end 42.5 38.350057) (width 0.2) (layer "F.Cu") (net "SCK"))
 (via (at 42.5 44) (size 0.6) (drill 0.3) (layers "F.Cu" "B.Cu") (capping no) (covering (front no) (back no))
  (plugging (front no) (back no)) (filling no) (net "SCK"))
 (segment (start 43.3 43.2) (end 48.265 43.2) (width 0.2) (layer "B.Cu") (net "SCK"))
 (segment (start 48.265 43.2) (end 50.185 41.28) (width 0.2) (layer "B.Cu") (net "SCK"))
 (segment (start 42.5 44) (end 43.3 43.2) (width 0.2) (layer "B.Cu") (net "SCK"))
 (segment (start 46.165 37.8) (end 44.1 37.8) (width 0.2) (layer "F.Cu") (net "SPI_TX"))
 (segment (start 43.5 47) (end 47.005 47) (width 0.2) (layer "F.Cu") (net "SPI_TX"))
 (segment (start 44.1 37.8) (end 43.5 38.4) (width 0.2) (layer "F.Cu") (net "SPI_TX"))
 (segment (start 47.005 47) (end 50.185 43.82) (width 0.2) (layer "F.Cu") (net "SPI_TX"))
 (segment (start 43.5 38.4) (end 43.5 47) (width 0.2) (layer "F.Cu") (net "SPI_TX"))
 (segment (start 33.835 36.2) (end 37.99 36.2) (width 0.2) (layer "F.Cu") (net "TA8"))
 (segment (start 37.99 36.2) (end 42.79 31.4) (width 0.2) (layer "F.Cu") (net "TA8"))
 (segment (start 43.49 30.7) (end 45.45 30.7) (width 0.2) (layer "F.Cu") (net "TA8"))
 (segment (start 45.45 30.7) (end 45.6 30.85) (width 0.2) (layer "F.Cu") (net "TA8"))
 (segment (start 42.79 31.4) (end 43.49 30.7) (width 0.2) (layer "F.Cu") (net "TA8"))
 (segment (start 33.835 41.4) (end 33.835 41.8) (width 0.5) (layer "F.Cu") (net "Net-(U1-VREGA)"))
 (segment (start 33.835 41.4) (end 32.7 41.4) (width 0.5) (layer "F.Cu") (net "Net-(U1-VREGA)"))
 (segment (start 32.7 41.4) (end 32.2 41.9) (width 0.5) (layer "F.Cu") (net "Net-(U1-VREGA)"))
 (segment (start 32.2 41.9) (end 32.2 44.45) (width 0.5) (layer "F.Cu") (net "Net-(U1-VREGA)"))
 (segment (start 32.2 44.45) (end 33 45.25) (width 0.5) (layer "F.Cu") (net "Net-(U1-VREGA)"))
 (segment (start 33.835 41) (end 33.835 41.4) (width 0.5) (layer "F.Cu") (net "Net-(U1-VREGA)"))
 (segment (start 37.21 31.4) (end 36.589 30.779) (width 0.2) (layer "F.Cu") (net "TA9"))
 (segment (start 33.835 35.4) (end 34.8 35.4) (width 0.2) (layer "F.Cu") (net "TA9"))
 (segment (start 37.21 32.99) (end 37.21 31.4) (width 0.2) (layer "F.Cu") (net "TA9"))
 (segment (start 36.589 30.779) (end 34.471 30.779) (width 0.2) (layer "F.Cu") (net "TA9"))
 (segment (start 34.8 35.4) (end 37.21 32.99) (width 0.2) (layer "F.Cu") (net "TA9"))
 (segment (start 34.471 30.779) (end 34.4 30.85) (width 0.2) (layer "F.Cu") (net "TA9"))
 (segment (start 46.165 41.8) (end 46.565 41.4) (width 0.5) (layer "F.Cu") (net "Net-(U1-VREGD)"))
 (segment (start 46.565 41.4) (end 47.475 41.4) (width 0.5) (layer "F.Cu") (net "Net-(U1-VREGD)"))
 (segment (start 46.165 41.4) (end 46.165 41) (width 0.5) (layer "F.Cu") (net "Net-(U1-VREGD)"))
 (segment (start 47.475 41.4) (end 48.1 42.025) (width 0.5) (layer "F.Cu") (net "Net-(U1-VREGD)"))
 (segment (start 46.165 41.8) (end 46.165 41.4) (width 0.5) (layer "F.Cu") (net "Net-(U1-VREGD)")))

